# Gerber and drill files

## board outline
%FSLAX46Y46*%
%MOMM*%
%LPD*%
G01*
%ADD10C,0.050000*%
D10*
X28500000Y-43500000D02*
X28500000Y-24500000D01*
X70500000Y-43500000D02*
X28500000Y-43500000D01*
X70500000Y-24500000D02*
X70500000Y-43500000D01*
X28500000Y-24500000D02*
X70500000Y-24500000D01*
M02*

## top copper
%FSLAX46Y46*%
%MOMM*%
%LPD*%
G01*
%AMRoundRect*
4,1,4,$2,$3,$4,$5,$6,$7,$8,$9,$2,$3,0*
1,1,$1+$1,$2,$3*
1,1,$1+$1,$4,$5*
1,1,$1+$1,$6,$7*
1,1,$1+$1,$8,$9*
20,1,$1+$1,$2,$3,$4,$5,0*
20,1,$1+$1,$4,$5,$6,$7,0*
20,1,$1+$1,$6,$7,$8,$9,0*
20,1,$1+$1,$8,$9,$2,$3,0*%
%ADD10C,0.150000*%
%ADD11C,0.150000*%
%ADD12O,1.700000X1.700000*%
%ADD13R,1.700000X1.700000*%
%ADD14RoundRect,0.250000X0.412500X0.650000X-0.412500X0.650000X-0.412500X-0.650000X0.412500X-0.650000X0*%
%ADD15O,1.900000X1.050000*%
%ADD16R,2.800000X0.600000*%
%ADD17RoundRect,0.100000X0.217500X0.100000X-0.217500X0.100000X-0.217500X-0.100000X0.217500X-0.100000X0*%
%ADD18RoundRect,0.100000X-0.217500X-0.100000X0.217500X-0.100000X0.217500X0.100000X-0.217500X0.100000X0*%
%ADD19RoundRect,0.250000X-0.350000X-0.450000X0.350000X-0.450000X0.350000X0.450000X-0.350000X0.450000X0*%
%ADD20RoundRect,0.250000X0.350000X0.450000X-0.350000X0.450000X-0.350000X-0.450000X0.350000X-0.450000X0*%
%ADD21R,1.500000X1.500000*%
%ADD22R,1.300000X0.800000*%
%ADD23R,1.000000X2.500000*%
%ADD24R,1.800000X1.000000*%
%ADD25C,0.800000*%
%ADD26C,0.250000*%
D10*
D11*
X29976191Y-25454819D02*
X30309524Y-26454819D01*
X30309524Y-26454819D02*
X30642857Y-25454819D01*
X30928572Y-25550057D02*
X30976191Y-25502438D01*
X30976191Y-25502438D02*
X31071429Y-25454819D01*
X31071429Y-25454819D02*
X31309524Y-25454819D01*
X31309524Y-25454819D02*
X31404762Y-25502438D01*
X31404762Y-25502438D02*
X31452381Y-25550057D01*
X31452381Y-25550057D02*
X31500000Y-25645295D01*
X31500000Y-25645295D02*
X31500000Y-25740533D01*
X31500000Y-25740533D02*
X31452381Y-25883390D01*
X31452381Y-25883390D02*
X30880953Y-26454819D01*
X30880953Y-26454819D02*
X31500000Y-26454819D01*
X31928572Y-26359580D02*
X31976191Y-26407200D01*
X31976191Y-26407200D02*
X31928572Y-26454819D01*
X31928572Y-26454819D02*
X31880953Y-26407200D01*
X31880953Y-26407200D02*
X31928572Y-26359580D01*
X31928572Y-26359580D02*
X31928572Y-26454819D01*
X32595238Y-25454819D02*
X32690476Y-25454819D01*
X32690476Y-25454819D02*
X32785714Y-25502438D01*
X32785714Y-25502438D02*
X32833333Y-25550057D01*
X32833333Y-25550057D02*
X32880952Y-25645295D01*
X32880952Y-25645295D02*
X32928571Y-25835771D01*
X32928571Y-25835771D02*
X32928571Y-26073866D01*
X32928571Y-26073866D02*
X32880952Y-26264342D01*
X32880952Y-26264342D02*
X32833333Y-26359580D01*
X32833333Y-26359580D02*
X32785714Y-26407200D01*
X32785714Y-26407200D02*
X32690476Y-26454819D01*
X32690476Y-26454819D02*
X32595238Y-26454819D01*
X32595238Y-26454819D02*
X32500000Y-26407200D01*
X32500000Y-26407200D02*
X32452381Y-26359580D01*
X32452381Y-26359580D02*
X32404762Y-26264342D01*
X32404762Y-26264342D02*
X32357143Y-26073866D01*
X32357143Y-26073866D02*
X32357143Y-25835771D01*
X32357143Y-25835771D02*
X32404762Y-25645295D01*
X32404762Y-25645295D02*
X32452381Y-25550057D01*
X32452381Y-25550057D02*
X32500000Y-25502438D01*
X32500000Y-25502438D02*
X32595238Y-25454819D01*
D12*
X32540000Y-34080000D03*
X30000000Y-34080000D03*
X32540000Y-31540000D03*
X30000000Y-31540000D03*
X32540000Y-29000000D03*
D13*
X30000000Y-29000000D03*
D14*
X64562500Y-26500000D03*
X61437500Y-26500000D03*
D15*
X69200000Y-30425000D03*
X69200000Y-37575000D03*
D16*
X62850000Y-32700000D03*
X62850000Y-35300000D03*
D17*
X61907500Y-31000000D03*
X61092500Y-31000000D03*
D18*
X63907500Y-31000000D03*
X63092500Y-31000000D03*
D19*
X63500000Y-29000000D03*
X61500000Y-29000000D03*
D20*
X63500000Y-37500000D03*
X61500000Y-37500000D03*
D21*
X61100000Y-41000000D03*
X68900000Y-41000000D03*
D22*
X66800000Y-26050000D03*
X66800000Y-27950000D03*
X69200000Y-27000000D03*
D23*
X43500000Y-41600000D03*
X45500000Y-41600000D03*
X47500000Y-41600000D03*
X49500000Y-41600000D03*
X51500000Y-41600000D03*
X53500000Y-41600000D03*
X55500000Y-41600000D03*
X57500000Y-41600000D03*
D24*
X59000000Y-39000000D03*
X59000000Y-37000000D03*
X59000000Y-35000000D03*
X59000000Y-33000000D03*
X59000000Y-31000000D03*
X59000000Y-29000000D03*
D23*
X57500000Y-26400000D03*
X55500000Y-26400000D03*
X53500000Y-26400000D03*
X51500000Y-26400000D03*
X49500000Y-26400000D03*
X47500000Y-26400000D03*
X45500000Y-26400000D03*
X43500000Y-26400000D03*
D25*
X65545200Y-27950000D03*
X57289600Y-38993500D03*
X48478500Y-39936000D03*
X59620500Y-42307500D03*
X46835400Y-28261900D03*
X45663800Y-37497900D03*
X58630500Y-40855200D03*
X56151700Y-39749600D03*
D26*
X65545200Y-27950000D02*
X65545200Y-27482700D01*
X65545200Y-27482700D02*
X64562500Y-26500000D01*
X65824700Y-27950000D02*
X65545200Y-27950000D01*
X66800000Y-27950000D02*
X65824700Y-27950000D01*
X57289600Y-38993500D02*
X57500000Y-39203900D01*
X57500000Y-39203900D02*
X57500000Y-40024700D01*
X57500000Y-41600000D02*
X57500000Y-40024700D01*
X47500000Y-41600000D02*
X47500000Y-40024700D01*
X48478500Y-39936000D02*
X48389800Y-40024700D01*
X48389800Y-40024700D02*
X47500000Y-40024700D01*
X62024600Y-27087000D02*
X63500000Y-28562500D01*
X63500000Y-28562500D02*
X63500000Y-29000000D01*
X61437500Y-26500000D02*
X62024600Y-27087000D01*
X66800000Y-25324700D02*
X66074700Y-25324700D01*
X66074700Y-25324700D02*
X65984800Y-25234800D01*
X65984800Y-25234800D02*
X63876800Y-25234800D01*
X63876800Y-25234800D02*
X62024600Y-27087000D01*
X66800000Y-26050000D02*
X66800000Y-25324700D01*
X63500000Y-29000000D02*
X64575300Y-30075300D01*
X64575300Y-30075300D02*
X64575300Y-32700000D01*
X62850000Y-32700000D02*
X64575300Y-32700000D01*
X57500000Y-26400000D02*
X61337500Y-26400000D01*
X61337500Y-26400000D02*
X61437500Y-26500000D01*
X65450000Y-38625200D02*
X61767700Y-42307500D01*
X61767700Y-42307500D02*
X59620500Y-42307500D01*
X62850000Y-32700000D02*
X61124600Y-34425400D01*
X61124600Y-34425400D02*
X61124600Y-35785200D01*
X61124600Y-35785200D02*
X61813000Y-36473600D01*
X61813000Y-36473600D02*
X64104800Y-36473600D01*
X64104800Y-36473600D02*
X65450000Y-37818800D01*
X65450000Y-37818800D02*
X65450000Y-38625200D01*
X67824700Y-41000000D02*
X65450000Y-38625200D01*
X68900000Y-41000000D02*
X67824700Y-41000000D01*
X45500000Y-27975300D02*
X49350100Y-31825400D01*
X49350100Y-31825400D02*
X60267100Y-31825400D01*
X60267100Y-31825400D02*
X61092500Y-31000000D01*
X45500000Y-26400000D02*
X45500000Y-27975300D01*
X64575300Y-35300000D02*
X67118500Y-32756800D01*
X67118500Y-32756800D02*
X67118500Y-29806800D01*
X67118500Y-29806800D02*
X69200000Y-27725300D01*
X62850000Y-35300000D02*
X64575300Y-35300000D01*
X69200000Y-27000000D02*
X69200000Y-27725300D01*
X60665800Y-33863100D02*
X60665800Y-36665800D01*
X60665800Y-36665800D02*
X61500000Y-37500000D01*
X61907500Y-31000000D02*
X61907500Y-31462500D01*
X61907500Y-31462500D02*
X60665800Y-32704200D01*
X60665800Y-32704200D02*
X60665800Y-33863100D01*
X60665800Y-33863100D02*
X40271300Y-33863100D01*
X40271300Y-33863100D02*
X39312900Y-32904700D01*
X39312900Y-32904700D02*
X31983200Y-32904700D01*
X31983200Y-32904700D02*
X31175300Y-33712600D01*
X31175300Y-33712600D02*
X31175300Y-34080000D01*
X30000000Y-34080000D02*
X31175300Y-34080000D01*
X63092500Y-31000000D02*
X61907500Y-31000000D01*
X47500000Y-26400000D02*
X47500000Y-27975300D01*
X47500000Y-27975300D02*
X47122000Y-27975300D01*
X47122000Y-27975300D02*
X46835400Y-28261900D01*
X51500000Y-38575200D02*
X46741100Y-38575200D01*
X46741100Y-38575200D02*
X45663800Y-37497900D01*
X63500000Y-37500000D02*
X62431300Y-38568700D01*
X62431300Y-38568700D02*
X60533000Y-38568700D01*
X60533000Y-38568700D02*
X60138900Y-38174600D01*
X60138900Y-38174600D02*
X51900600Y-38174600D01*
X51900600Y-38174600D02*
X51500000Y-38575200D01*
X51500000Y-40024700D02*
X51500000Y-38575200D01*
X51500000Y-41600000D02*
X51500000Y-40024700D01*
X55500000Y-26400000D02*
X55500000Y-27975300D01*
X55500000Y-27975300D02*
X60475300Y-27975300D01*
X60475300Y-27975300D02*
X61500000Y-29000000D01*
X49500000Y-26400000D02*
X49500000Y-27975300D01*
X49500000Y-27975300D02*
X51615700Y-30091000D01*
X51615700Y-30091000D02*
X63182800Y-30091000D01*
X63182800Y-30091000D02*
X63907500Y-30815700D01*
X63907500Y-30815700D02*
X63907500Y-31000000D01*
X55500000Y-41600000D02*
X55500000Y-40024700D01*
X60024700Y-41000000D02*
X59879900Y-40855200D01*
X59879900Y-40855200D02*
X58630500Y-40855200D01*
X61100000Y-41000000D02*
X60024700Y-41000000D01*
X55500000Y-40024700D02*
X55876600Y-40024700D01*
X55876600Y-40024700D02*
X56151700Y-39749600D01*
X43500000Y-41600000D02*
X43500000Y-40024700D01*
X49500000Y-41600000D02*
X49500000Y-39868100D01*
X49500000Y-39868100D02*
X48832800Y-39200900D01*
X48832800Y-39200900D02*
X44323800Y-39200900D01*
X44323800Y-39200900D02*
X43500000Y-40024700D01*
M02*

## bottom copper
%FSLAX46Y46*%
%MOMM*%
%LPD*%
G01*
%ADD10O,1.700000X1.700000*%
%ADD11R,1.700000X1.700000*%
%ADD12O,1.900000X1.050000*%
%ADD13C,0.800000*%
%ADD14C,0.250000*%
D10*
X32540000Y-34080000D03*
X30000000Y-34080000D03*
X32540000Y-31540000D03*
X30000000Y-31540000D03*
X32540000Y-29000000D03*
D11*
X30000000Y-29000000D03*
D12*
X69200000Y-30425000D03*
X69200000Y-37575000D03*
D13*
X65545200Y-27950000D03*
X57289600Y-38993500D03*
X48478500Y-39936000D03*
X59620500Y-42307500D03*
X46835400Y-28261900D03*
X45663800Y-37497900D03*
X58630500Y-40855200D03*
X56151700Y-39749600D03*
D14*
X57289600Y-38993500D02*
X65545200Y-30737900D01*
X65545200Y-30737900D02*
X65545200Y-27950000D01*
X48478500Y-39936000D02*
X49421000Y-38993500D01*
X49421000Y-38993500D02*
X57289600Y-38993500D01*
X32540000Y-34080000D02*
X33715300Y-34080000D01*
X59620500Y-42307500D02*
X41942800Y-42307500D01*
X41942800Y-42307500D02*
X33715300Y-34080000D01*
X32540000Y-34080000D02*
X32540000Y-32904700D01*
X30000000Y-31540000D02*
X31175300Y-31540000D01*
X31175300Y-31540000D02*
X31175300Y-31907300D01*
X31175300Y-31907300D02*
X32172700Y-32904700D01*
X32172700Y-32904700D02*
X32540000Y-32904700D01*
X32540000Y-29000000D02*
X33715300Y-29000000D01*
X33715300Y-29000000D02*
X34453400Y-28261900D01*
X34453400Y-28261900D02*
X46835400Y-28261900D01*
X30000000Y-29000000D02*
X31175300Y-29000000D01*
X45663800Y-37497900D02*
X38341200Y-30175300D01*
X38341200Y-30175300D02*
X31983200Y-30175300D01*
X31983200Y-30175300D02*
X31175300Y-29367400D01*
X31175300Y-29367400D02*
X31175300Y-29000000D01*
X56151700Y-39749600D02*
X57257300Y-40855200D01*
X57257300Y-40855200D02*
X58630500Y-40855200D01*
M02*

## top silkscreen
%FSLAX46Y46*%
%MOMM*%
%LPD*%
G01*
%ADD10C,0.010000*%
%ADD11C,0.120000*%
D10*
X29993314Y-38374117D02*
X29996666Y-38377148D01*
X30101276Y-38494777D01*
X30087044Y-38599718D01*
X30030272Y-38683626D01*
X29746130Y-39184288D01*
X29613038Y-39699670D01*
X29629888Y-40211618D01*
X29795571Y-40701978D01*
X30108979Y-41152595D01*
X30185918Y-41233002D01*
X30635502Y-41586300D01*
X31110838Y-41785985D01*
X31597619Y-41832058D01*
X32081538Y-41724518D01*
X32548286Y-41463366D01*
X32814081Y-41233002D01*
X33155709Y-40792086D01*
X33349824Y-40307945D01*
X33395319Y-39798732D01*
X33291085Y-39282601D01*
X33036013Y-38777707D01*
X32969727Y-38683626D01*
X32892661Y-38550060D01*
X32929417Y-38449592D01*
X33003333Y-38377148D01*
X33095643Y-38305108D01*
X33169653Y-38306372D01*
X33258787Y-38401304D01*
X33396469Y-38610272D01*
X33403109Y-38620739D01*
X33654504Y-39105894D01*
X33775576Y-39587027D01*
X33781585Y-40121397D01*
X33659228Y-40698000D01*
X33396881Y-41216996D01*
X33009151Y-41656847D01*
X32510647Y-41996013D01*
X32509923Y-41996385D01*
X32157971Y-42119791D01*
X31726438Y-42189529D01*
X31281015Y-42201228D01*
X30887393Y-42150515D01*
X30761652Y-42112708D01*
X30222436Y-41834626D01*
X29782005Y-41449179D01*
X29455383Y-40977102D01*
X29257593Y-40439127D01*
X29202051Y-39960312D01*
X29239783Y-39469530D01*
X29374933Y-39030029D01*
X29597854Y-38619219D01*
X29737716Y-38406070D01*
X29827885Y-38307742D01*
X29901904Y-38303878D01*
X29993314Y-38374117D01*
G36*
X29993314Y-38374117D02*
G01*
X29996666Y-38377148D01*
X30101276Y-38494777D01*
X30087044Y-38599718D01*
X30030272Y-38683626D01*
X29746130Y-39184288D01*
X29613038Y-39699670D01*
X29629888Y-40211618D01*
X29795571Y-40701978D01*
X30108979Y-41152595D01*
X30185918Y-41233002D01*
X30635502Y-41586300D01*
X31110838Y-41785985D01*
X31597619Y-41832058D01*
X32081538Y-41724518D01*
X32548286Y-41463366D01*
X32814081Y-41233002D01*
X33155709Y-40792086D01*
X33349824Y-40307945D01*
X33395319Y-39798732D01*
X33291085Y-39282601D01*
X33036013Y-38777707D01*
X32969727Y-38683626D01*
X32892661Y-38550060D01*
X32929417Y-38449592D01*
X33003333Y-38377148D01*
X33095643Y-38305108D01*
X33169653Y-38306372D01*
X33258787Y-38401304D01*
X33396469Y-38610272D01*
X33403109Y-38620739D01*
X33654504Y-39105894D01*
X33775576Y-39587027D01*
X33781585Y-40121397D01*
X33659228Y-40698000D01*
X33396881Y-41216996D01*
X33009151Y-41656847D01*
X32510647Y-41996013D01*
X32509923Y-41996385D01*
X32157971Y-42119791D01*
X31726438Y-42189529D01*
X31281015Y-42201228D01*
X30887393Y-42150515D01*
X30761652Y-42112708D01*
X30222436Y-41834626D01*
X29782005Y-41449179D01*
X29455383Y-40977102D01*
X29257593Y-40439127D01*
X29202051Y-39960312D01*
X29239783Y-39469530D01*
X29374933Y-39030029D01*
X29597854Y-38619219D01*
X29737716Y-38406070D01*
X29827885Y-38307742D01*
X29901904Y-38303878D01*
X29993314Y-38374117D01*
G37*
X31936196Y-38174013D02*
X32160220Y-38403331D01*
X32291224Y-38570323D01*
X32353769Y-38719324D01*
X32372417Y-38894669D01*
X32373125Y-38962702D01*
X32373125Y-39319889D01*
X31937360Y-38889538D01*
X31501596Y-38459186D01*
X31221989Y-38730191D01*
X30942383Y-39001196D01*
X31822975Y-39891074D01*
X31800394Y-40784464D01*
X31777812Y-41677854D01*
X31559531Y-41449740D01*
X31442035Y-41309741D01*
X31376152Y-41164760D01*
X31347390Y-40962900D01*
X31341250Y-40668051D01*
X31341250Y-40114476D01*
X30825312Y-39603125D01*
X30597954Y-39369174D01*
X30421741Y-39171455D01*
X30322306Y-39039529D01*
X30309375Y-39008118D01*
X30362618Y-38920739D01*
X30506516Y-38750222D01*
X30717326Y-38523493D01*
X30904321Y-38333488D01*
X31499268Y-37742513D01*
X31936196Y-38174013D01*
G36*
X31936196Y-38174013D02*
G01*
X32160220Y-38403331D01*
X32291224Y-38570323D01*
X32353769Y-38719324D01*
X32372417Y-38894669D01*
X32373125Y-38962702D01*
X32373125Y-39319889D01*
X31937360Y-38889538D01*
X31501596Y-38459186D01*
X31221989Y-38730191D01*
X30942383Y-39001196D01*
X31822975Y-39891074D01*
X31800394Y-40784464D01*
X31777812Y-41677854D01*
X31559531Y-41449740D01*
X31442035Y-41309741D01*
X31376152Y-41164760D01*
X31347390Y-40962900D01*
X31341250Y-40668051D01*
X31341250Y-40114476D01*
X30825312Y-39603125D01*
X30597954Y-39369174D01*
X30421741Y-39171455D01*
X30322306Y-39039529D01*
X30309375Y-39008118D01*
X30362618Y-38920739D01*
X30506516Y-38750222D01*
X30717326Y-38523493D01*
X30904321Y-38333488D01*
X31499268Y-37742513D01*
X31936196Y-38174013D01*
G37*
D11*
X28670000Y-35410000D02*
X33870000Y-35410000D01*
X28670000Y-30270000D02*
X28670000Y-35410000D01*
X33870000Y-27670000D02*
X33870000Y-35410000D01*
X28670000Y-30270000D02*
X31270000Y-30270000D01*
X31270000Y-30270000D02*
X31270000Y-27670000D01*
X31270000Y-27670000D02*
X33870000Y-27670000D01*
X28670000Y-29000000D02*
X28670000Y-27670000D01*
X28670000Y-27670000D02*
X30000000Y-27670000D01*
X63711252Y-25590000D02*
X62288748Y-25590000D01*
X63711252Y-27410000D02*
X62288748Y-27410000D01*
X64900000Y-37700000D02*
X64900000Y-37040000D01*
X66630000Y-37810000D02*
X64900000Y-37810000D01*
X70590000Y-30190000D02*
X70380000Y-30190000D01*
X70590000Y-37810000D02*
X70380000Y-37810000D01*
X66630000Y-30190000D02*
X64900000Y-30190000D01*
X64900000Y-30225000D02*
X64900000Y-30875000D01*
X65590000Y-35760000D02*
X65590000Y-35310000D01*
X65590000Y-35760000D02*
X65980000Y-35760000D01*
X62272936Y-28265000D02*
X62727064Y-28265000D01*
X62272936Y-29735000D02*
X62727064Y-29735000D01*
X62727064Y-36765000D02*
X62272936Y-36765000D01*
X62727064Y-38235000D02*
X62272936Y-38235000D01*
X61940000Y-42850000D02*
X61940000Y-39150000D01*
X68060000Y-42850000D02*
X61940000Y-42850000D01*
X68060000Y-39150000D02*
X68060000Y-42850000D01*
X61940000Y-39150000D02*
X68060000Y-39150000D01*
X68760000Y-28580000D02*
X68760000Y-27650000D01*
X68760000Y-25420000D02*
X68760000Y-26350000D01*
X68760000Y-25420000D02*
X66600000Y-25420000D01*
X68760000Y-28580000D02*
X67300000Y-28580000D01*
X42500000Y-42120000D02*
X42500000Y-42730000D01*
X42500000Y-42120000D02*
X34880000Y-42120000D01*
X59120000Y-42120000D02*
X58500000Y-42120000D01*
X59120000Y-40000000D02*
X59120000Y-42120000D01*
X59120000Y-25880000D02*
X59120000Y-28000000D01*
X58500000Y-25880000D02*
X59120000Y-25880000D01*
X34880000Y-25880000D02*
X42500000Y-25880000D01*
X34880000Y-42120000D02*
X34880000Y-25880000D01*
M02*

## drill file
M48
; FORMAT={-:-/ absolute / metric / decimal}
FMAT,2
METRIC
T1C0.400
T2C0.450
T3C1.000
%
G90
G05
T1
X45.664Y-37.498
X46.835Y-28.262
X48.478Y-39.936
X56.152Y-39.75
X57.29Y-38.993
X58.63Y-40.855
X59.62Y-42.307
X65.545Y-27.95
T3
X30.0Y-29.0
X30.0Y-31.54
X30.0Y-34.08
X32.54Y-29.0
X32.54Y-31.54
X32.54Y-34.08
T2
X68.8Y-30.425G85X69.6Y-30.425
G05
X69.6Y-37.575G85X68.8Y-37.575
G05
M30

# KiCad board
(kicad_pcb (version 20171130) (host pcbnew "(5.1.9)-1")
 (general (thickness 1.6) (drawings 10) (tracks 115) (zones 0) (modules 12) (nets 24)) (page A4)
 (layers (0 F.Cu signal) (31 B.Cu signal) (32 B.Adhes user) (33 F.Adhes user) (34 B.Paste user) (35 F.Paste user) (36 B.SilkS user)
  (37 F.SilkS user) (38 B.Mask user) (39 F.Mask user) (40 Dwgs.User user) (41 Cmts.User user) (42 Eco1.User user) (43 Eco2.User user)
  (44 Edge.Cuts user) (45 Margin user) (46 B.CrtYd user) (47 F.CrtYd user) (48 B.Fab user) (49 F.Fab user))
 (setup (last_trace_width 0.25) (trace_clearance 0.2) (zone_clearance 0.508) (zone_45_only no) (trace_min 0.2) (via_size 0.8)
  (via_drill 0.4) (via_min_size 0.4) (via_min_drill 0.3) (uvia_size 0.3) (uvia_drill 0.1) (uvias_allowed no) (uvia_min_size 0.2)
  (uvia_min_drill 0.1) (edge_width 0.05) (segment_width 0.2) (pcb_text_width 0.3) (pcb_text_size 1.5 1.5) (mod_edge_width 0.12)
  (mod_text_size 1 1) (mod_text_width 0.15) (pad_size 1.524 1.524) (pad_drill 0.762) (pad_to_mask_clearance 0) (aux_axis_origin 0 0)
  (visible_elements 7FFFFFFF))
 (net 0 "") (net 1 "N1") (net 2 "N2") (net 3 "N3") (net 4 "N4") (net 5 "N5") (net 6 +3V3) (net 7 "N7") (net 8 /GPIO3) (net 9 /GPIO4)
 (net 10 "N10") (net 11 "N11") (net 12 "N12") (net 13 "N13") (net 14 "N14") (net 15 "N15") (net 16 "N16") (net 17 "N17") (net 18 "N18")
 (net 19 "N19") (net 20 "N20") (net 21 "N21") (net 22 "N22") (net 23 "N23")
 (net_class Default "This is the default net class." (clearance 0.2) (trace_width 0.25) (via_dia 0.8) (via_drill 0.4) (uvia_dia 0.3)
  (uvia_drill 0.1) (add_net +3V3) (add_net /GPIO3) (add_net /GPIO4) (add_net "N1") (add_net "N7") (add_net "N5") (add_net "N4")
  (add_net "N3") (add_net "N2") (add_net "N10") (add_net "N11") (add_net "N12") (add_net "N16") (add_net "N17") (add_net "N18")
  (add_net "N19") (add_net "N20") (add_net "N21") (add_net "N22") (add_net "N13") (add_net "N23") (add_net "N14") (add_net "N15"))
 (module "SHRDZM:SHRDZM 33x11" (layer B.Cu) (at 51 31.5 180)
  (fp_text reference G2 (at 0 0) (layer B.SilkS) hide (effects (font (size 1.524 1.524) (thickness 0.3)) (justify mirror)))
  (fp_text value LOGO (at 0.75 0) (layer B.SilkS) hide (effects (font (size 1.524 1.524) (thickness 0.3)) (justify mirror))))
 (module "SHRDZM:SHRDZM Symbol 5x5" (layer F.Cu) (at 31.5 40)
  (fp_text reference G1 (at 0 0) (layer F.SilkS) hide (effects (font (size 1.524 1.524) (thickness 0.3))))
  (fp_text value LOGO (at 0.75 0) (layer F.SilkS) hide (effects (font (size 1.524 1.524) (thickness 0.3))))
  (fp_poly
   (pts (xy -1.506686 -1.625883) (xy -1.503334 -1.622852) (xy -1.398724 -1.505223) (xy -1.412956 -1.400282) (xy -1.469728 -1.316374)
    (xy -1.75387 -0.815712) (xy -1.886962 -0.30033) (xy -1.870112 0.211618) (xy -1.704429 0.701978) (xy -1.391021 1.152595)
    (xy -1.314082 1.233002) (xy -0.864498 1.5863) (xy -0.389162 1.785985) (xy 0.097619 1.832058) (xy 0.581538 1.724518)
    (xy 1.048286 1.463366) (xy 1.314081 1.233002) (xy 1.655709 0.792086) (xy 1.849824 0.307945) (xy 1.895319 -0.201268)
    (xy 1.791085 -0.717399) (xy 1.536013 -1.222293) (xy 1.469727 -1.316374) (xy 1.392661 -1.44994) (xy 1.429417 -1.550408)
    (xy 1.503333 -1.622852) (xy 1.595643 -1.694892) (xy 1.669653 -1.693628) (xy 1.758787 -1.598696) (xy 1.896469 -1.389728)
    (xy 1.903109 -1.379261) (xy 2.154504 -0.894106) (xy 2.275576 -0.412973) (xy 2.281585 0.121397) (xy 2.159228 0.698)
    (xy 1.896881 1.216996) (xy 1.509151 1.656847) (xy 1.010647 1.996013) (xy 1.009923 1.996385) (xy 0.657971 2.119791)
    (xy 0.226438 2.189529) (xy -0.218985 2.201228) (xy -0.612607 2.150515) (xy -0.738348 2.112708) (xy -1.277564 1.834626)
    (xy -1.717995 1.449179) (xy -2.044617 0.977102) (xy -2.242407 0.439127) (xy -2.297949 -0.039688) (xy -2.260217 -0.53047)
    (xy -2.125067 -0.969971) (xy -1.902146 -1.380781) (xy -1.762284 -1.59393) (xy -1.672115 -1.692258) (xy -1.598096 -1.696122)
    (xy -1.506686 -1.625883))
   (layer F.SilkS) (width 0.01))
  (fp_poly
   (pts (xy 0.436196 -1.825987) (xy 0.66022 -1.596669) (xy 0.791224 -1.429677) (xy 0.853769 -1.280676) (xy 0.872417 -1.105331)
    (xy 0.873125 -1.037298) (xy 0.873125 -0.680111) (xy 0.43736 -1.110462) (xy 0.001596 -1.540814) (xy -0.278011 -1.269809)
    (xy -0.557617 -0.998804) (xy 0.322975 -0.108926) (xy 0.300394 0.784464) (xy 0.277812 1.677854) (xy 0.059531 1.44974)
    (xy -0.057965 1.309741) (xy -0.123848 1.16476) (xy -0.15261 0.9629) (xy -0.15875 0.668051) (xy -0.15875 0.114476)
    (xy -0.674688 -0.396875) (xy -0.902046 -0.630826) (xy -1.078259 -0.828545) (xy -1.177694 -0.960471) (xy -1.190625 -0.991882)
    (xy -1.137382 -1.079261) (xy -0.993484 -1.249778) (xy -0.782674 -1.476507) (xy -0.595679 -1.666512) (xy -0.000732 -2.257487)
    (xy 0.436196 -1.825987))
   (layer F.SilkS) (width 0.01)))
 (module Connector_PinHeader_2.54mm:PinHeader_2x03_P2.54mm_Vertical (layer F.Cu) (at 30 29)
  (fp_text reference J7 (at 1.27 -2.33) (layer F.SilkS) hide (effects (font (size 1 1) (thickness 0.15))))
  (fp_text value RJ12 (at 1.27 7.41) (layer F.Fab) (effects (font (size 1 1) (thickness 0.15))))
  (fp_line (start -1.33 6.41) (end 3.87 6.41) (layer F.SilkS) (width 0.12))
  (fp_line (start -1.33 1.27) (end -1.33 6.41) (layer F.SilkS) (width 0.12))
  (fp_line (start 3.87 -1.33) (end 3.87 6.41) (layer F.SilkS) (width 0.12))
  (fp_line (start -1.33 1.27) (end 1.27 1.27) (layer F.SilkS) (width 0.12))
  (fp_line (start 1.27 1.27) (end 1.27 -1.33) (layer F.SilkS) (width 0.12))
  (fp_line (start 1.27 -1.33) (end 3.87 -1.33) (layer F.SilkS) (width 0.12))
  (fp_line (start -1.33 0) (end -1.33 -1.33) (layer F.SilkS) (width 0.12))
  (fp_line (start -1.33 -1.33) (end 0 -1.33) (layer F.SilkS) (width 0.12))
  (pad 6 thru_hole oval (at 2.54 5.08) (size 1.7 1.7) (drill 1) (layers *.Cu *.Mask) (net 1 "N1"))
  (pad 5 thru_hole oval (at 0 5.08) (size 1.7 1.7) (drill 1) (layers *.Cu *.Mask) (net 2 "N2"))
  (pad 4 thru_hole oval (at 2.54 2.54) (size 1.7 1.7) (drill 1) (layers *.Cu *.Mask) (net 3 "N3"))
  (pad 3 thru_hole oval (at 0 2.54) (size 1.7 1.7) (drill 1) (layers *.Cu *.Mask) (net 1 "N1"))
  (pad 2 thru_hole oval (at 2.54 0) (size 1.7 1.7) (drill 1) (layers *.Cu *.Mask) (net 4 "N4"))
  (pad 1 thru_hole rect (at 0 0) (size 1.7 1.7) (drill 1) (layers *.Cu *.Mask) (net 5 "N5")))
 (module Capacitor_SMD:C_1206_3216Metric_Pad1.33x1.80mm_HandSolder (layer F.Cu) (at 63 26.5 180)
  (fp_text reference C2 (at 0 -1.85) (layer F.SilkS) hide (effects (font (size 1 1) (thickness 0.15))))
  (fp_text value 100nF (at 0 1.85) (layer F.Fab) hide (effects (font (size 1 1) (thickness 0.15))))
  (fp_line (start -0.711252 0.91) (end 0.711252 0.91) (layer F.SilkS) (width 0.12))
  (fp_line (start -0.711252 -0.91) (end 0.711252 -0.91) (layer F.SilkS) (width 0.12))
  (pad 1 smd roundrect (at -1.5625 0 180) (size 1.325 1.8) (layers F.Cu F.Paste F.Mask) (roundrect_rratio 0.188679) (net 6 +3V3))
  (pad 2 smd roundrect (at 1.5625 0 180) (size 1.325 1.8) (layers F.Cu F.Paste F.Mask) (roundrect_rratio 0.188679) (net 1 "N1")))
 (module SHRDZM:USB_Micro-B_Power (layer F.Cu) (at 68 34 90)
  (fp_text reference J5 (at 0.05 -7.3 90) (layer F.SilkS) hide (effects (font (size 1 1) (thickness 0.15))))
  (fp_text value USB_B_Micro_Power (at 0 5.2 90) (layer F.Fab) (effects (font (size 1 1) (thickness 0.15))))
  (fp_line (start -3.7 -3.1) (end -3.04 -3.1) (layer F.SilkS) (width 0.12))
  (fp_line (start -3.81 -1.37) (end -3.81 -3.1) (layer F.SilkS) (width 0.12))
  (fp_line (start 3.81 2.59) (end 3.81 2.38) (layer F.SilkS) (width 0.12))
  (fp_line (start -3.81 2.59) (end -3.81 2.38) (layer F.SilkS) (width 0.12))
  (fp_line (start 3.81 -1.37) (end 3.81 -3.1) (layer F.SilkS) (width 0.12))
  (fp_line (start 3.775 -3.1) (end 3.125 -3.1) (layer F.SilkS) (width 0.12))
  (fp_line (start -1.76 -2.41) (end -1.31 -2.41) (layer F.SilkS) (width 0.12))
  (fp_line (start -1.76 -2.41) (end -1.76 -2.02) (layer F.SilkS) (width 0.12))
  (pad "" thru_hole oval (at 3.575 1.2 90) (size 1.05 1.9) (drill oval 0.45 1.25) (layers *.Cu *.Mask))
  (pad "" thru_hole oval (at -3.575 1.2 270) (size 1.05 1.9) (drill oval 0.45 1.25) (layers *.Cu *.Mask))
  (pad 5 smd rect (at 1.3 -5.15 90) (size 0.6 2.8) (layers F.Cu F.Paste F.Mask) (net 1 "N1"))
  (pad 1 smd rect (at -1.3 -5.15 90) (size 0.6 2.8) (layers F.Cu F.Paste F.Mask) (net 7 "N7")))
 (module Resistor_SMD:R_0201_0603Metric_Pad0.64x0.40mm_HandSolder (layer F.Cu) (at 61.5 31 180)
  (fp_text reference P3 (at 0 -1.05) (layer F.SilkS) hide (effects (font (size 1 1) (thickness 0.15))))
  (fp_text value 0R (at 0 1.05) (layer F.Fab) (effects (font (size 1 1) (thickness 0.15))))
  (pad "" smd roundrect (at -0.4325 0 180) (size 0.458 0.36) (layers F.Paste) (roundrect_rratio 0.25))
  (pad "" smd roundrect (at 0.4325 0 180) (size 0.458 0.36) (layers F.Paste) (roundrect_rratio 0.25))
  (pad 1 smd roundrect (at -0.4075 0 180) (size 0.635 0.4) (layers F.Cu F.Mask) (roundrect_rratio 0.25) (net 2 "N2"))
  (pad 2 smd roundrect (at 0.4075 0 180) (size 0.635 0.4) (layers F.Cu F.Mask) (roundrect_rratio 0.25) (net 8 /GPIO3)))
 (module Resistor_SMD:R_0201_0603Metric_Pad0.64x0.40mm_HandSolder (layer F.Cu) (at 63.5 31)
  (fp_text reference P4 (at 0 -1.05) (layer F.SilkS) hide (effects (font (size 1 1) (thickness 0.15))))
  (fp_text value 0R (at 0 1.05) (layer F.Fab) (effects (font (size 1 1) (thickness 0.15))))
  (pad 2 smd roundrect (at 0.4075 0) (size 0.635 0.4) (layers F.Cu F.Mask) (roundrect_rratio 0.25) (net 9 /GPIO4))
  (pad 1 smd roundrect (at -0.4075 0) (size 0.635 0.4) (layers F.Cu F.Mask) (roundrect_rratio 0.25) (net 2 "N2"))
  (pad "" smd roundrect (at 0.4325 0) (size 0.458 0.36) (layers F.Paste) (roundrect_rratio 0.25))
  (pad "" smd roundrect (at -0.4325 0) (size 0.458 0.36) (layers F.Paste) (roundrect_rratio 0.25)))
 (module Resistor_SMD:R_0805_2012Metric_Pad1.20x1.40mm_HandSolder (layer F.Cu) (at 62.5 29)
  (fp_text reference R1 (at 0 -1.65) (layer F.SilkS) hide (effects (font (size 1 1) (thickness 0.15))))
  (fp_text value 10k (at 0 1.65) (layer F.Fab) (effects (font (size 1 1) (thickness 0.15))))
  (fp_line (start -0.227064 -0.735) (end 0.227064 -0.735) (layer F.SilkS) (width 0.12))
  (fp_line (start -0.227064 0.735) (end 0.227064 0.735) (layer F.SilkS) (width 0.12))
  (pad 2 smd roundrect (at 1 0) (size 1.2 1.4) (layers F.Cu F.Paste F.Mask) (roundrect_rratio 0.208333) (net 1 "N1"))
  (pad 1 smd roundrect (at -1 0) (size 1.2 1.4) (layers F.Cu F.Paste F.Mask) (roundrect_rratio 0.208333) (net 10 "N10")))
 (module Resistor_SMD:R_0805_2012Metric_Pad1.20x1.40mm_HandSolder (layer F.Cu) (at 62.5 37.5 180)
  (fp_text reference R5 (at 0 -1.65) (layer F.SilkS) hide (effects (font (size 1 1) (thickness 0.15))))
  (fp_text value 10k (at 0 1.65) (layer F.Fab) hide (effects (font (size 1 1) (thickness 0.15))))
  (fp_line (start -0.227064 0.735) (end 0.227064 0.735) (layer F.SilkS) (width 0.12))
  (fp_line (start -0.227064 -0.735) (end 0.227064 -0.735) (layer F.SilkS) (width 0.12))
  (pad 1 smd roundrect (at -1 0 180) (size 1.2 1.4) (layers F.Cu F.Paste F.Mask) (roundrect_rratio 0.208333) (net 5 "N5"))
  (pad 2 smd roundrect (at 1 0 180) (size 1.2 1.4) (layers F.Cu F.Paste F.Mask) (roundrect_rratio 0.208333) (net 2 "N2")))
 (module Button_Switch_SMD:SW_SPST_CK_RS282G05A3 (layer F.Cu) (at 65 41)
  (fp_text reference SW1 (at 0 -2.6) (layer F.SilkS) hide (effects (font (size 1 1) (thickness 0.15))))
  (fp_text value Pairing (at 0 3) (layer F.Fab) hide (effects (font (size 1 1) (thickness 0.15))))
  (fp_line (start -3.06 1.85) (end -3.06 -1.85) (layer F.SilkS) (width 0.12))
  (fp_line (start 3.06 1.85) (end -3.06 1.85) (layer F.SilkS) (width 0.12))
  (fp_line (start 3.06 -1.85) (end 3.06 1.85) (layer F.SilkS) (width 0.12))
  (fp_line (start -3.06 -1.85) (end 3.06 -1.85) (layer F.SilkS) (width 0.12))
  (pad 1 smd rect (at -3.9 0) (size 1.5 1.5) (layers F.Cu F.Paste F.Mask) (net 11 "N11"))
  (pad 2 smd rect (at 3.9 0) (size 1.5 1.5) (layers F.Cu F.Paste F.Mask) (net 1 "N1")))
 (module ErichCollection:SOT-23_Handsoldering (layer F.Cu) (at 68 27)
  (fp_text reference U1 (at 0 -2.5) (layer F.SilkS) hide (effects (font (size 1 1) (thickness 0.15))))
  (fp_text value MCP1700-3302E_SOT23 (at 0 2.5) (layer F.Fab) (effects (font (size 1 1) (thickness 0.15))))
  (fp_line (start 0.76 1.58) (end 0.76 0.65) (layer F.SilkS) (width 0.12))
  (fp_line (start 0.76 -1.58) (end 0.76 -0.65) (layer F.SilkS) (width 0.12))
  (fp_line (start 0.76 -1.58) (end -1.4 -1.58) (layer F.SilkS) (width 0.12))
  (fp_line (start 0.76 1.58) (end -0.7 1.58) (layer F.SilkS) (width 0.12))
  (pad 1 smd rect (at -1.2 -0.95) (size 1.3 0.8) (layers F.Cu F.Paste F.Mask) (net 1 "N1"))
  (pad 2 smd rect (at -1.2 0.95) (size 1.3 0.8) (layers F.Cu F.Paste F.Mask) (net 6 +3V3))
  (pad 3 smd rect (at 1.2 0) (size 1.3 0.8) (layers F.Cu F.Paste F.Mask) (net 7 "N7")))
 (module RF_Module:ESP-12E (layer F.Cu) (at 47 34 90)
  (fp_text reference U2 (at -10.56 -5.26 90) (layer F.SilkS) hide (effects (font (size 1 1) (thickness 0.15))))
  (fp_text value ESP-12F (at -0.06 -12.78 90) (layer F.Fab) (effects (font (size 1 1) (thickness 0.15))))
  (fp_line (start -8.12 -4.5) (end -8.73 -4.5) (layer F.SilkS) (width 0.12))
  (fp_line (start -8.12 -4.5) (end -8.12 -12.12) (layer F.SilkS) (width 0.12))
  (fp_line (start -8.12 12.12) (end -8.12 11.5) (layer F.SilkS) (width 0.12))
  (fp_line (start -6 12.12) (end -8.12 12.12) (layer F.SilkS) (width 0.12))
  (fp_line (start 8.12 12.12) (end 6 12.12) (layer F.SilkS) (width 0.12))
  (fp_line (start 8.12 11.5) (end 8.12 12.12) (layer F.SilkS) (width 0.12))
  (fp_line (start 8.12 -12.12) (end 8.12 -4.5) (layer F.SilkS) (width 0.12))
  (fp_line (start -8.12 -12.12) (end 8.12 -12.12) (layer F.SilkS) (width 0.12))
  (pad 1 smd rect (at -7.6 -3.5 90) (size 2.5 1) (layers F.Cu F.Paste F.Mask) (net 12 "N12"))
  (pad 2 smd rect (at -7.6 -1.5 90) (size 2.5 1) (layers F.Cu F.Paste F.Mask) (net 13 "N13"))
  (pad 3 smd rect (at -7.6 0.5 90) (size 2.5 1) (layers F.Cu F.Paste F.Mask) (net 6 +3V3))
  (pad 4 smd rect (at -7.6 2.5 90) (size 2.5 1) (layers F.Cu F.Paste F.Mask) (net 12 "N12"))
  (pad 5 smd rect (at -7.6 4.5 90) (size 2.5 1) (layers F.Cu F.Paste F.Mask) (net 5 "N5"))
  (pad 6 smd rect (at -7.6 6.5 90) (size 2.5 1) (layers F.Cu F.Paste F.Mask) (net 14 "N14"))
  (pad 7 smd rect (at -7.6 8.5 90) (size 2.5 1) (layers F.Cu F.Paste F.Mask) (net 11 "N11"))
  (pad 8 smd rect (at -7.6 10.5 90) (size 2.5 1) (layers F.Cu F.Paste F.Mask) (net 6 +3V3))
  (pad 9 smd rect (at -5 12 90) (size 1 1.8) (layers F.Cu F.Paste F.Mask) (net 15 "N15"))
  (pad 10 smd rect (at -3 12 90) (size 1 1.8) (layers F.Cu F.Paste F.Mask) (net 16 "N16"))
  (pad 11 smd rect (at -1 12 90) (size 1 1.8) (layers F.Cu F.Paste F.Mask) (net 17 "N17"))
  (pad 12 smd rect (at 1 12 90) (size 1 1.8) (layers F.Cu F.Paste F.Mask) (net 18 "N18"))
  (pad 13 smd rect (at 3 12 90) (size 1 1.8) (layers F.Cu F.Paste F.Mask) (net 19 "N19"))
  (pad 14 smd rect (at 5 12 90) (size 1 1.8) (layers F.Cu F.Paste F.Mask) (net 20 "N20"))
  (pad 15 smd rect (at 7.6 10.5 90) (size 2.5 1) (layers F.Cu F.Paste F.Mask) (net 1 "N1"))
  (pad 16 smd rect (at 7.6 8.5 90) (size 2.5 1) (layers F.Cu F.Paste F.Mask) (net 10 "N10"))
  (pad 17 smd rect (at 7.6 6.5 90) (size 2.5 1) (layers F.Cu F.Paste F.Mask) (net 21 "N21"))
  (pad 18 smd rect (at 7.6 4.5 90) (size 2.5 1) (layers F.Cu F.Paste F.Mask) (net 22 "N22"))
  (pad 19 smd rect (at 7.6 2.5 90) (size 2.5 1) (layers F.Cu F.Paste F.Mask) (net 9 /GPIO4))
  (pad 20 smd rect (at 7.6 0.5 90) (size 2.5 1) (layers F.Cu F.Paste F.Mask) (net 4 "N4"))
  (pad 21 smd rect (at 7.6 -1.5 90) (size 2.5 1) (layers F.Cu F.Paste F.Mask) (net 8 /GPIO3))
  (pad 22 smd rect (at 7.6 -3.5 90) (size 2.5 1) (layers F.Cu F.Paste F.Mask) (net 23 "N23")))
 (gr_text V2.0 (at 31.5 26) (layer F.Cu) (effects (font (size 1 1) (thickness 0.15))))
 (gr_line (start 28.5 43.5) (end 28.5 24.5) (layer Edge.Cuts) (width 0.05))
 (gr_line (start 70.5 43.5) (end 28.5 43.5) (layer Edge.Cuts) (width 0.05))
 (gr_line (start 70.5 24.5) (end 70.5 43.5) (layer Edge.Cuts) (width 0.05))
 (gr_line (start 28.5 24.5) (end 70.5 24.5) (layer Edge.Cuts) (width 0.05))
 (segment (start 65.5452 27.95) (end 65.5452 27.4827) (width 0.25) (layer F.Cu) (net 6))
 (segment (start 65.5452 27.4827) (end 64.5625 26.5) (width 0.25) (layer F.Cu) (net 6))
 (segment (start 65.8247 27.95) (end 65.5452 27.95) (width 0.25) (layer F.Cu) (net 6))
 (segment (start 57.2896 38.9935) (end 65.5452 30.7379) (width 0.25) (layer B.Cu) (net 6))
 (segment (start 65.5452 30.7379) (end 65.5452 27.95) (width 0.25) (layer B.Cu) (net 6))
 (segment (start 66.8 27.95) (end 65.8247 27.95) (width 0.25) (layer F.Cu) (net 6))
 (segment (start 57.2896 38.9935) (end 57.5 39.2039) (width 0.25) (layer F.Cu) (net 6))
 (segment (start 57.5 39.2039) (end 57.5 40.0247) (width 0.25) (layer F.Cu) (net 6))
 (segment (start 48.4785 39.936) (end 49.421 38.9935) (width 0.25) (layer B.Cu) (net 6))
 (segment (start 49.421 38.9935) (end 57.2896 38.9935) (width 0.25) (layer B.Cu) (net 6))
 (segment (start 57.5 41.6) (end 57.5 40.0247) (width 0.25) (layer F.Cu) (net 6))
 (segment (start 47.5 41.6) (end 47.5 40.0247) (width 0.25) (layer F.Cu) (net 6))
 (segment (start 48.4785 39.936) (end 48.3898 40.0247) (width 0.25) (layer F.Cu) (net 6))
 (segment (start 48.3898 40.0247) (end 47.5 40.0247) (width 0.25) (layer F.Cu) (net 6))
 (via (at 65.5452 27.95) (size 0.8) (layers F.Cu B.Cu) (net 6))
 (via (at 57.2896 38.9935) (size 0.8) (layers F.Cu B.Cu) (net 6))
 (via (at 48.4785 39.936) (size 0.8) (layers F.Cu B.Cu) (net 6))
 (segment (start 62.0246 27.087) (end 63.5 28.5625) (width 0.25) (layer F.Cu) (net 1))
 (segment (start 63.5 28.5625) (end 63.5 29) (width 0.25) (layer F.Cu) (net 1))
 (segment (start 61.4375 26.5) (end 62.0246 27.087) (width 0.25) (layer F.Cu) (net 1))
 (segment (start 66.8 25.3247) (end 66.0747 25.3247) (width 0.25) (layer F.Cu) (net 1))
 (segment (start 66.0747 25.3247) (end 65.9848 25.2348) (width 0.25) (layer F.Cu) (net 1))
 (segment (start 65.9848 25.2348) (end 63.8768 25.2348) (width 0.25) (layer F.Cu) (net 1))
 (segment (start 63.8768 25.2348) (end 62.0246 27.087) (width 0.25) (layer F.Cu) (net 1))
 (segment (start 66.8 26.05) (end 66.8 25.3247) (width 0.25) (layer F.Cu) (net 1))
 (segment (start 63.5 29) (end 64.5753 30.0753) (width 0.25) (layer F.Cu) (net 1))
 (segment (start 64.5753 30.0753) (end 64.5753 32.7) (width 0.25) (layer F.Cu) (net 1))
 (segment (start 62.85 32.7) (end 64.5753 32.7) (width 0.25) (layer F.Cu) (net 1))
 (segment (start 57.5 26.4) (end 61.3375 26.4) (width 0.25) (layer F.Cu) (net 1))
 (segment (start 61.3375 26.4) (end 61.4375 26.5) (width 0.25) (layer F.Cu) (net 1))
 (segment (start 65.45 38.6252) (end 61.7677 42.3075) (width 0.25) (layer F.Cu) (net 1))
 (segment (start 61.7677 42.3075) (end 59.6205 42.3075) (width 0.25) (layer F.Cu) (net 1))
 (segment (start 62.85 32.7) (end 61.1246 34.4254) (width 0.25) (layer F.Cu) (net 1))
 (segment (start 61.1246 34.4254) (end 61.1246 35.7852) (width 0.25) (layer F.Cu) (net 1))
 (segment (start 61.1246 35.7852) (end 61.813 36.4736) (width 0.25) (layer F.Cu) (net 1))
 (segment (start 61.813 36.4736) (end 64.1048 36.4736) (width 0.25) (layer F.Cu) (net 1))
 (segment (start 64.1048 36.4736) (end 65.45 37.8188) (width 0.25) (layer F.Cu) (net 1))
 (segment (start 65.45 37.8188) (end 65.45 38.6252) (width 0.25) (layer F.Cu) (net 1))
 (segment (start 67.8247 41) (end 65.45 38.6252) (width 0.25) (layer F.Cu) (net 1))
 (segment (start 32.54 34.08) (end 33.7153 34.08) (width 0.25) (layer B.Cu) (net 1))
 (segment (start 59.6205 42.3075) (end 41.9428 42.3075) (width 0.25) (layer B.Cu) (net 1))
 (segment (start 41.9428 42.3075) (end 33.7153 34.08) (width 0.25) (layer B.Cu) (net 1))
 (segment (start 68.9 41) (end 67.8247 41) (width 0.25) (layer F.Cu) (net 1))
 (segment (start 32.54 34.08) (end 32.54 32.9047) (width 0.25) (layer B.Cu) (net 1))
 (segment (start 30 31.54) (end 31.1753 31.54) (width 0.25) (layer B.Cu) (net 1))
 (segment (start 31.1753 31.54) (end 31.1753 31.9073) (width 0.25) (layer B.Cu) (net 1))
 (segment (start 31.1753 31.9073) (end 32.1727 32.9047) (width 0.25) (layer B.Cu) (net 1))
 (segment (start 32.1727 32.9047) (end 32.54 32.9047) (width 0.25) (layer B.Cu) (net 1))
 (via (at 59.6205 42.3075) (size 0.8) (layers F.Cu B.Cu) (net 1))
 (segment (start 45.5 27.9753) (end 49.3501 31.8254) (width 0.25) (layer F.Cu) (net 8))
 (segment (start 49.3501 31.8254) (end 60.2671 31.8254) (width 0.25) (layer F.Cu) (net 8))
 (segment (start 60.2671 31.8254) (end 61.0925 31) (width 0.25) (layer F.Cu) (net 8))
 (segment (start 45.5 26.4) (end 45.5 27.9753) (width 0.25) (layer F.Cu) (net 8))
 (segment (start 64.5753 35.3) (end 67.1185 32.7568) (width 0.25) (layer F.Cu) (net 7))
 (segment (start 67.1185 32.7568) (end 67.1185 29.8068) (width 0.25) (layer F.Cu) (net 7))
 (segment (start 67.1185 29.8068) (end 69.2 27.7253) (width 0.25) (layer F.Cu) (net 7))
 (segment (start 62.85 35.3) (end 64.5753 35.3) (width 0.25) (layer F.Cu) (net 7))
 (segment (start 69.2 27) (end 69.2 27.7253) (width 0.25) (layer F.Cu) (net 7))
 (segment (start 60.6658 33.8631) (end 60.6658 36.6658) (width 0.25) (layer F.Cu) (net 2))
 (segment (start 60.6658 36.6658) (end 61.5 37.5) (width 0.25) (layer F.Cu) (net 2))
 (segment (start 61.9075 31) (end 61.9075 31.4625) (width 0.25) (layer F.Cu) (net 2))
 (segment (start 61.9075 31.4625) (end 60.6658 32.7042) (width 0.25) (layer F.Cu) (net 2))
 (segment (start 60.6658 32.7042) (end 60.6658 33.8631) (width 0.25) (layer F.Cu) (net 2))
 (segment (start 60.6658 33.8631) (end 40.2713 33.8631) (width 0.25) (layer F.Cu) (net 2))
 (segment (start 40.2713 33.8631) (end 39.3129 32.9047) (width 0.25) (layer F.Cu) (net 2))
 (segment (start 39.3129 32.9047) (end 31.9832 32.9047) (width 0.25) (layer F.Cu) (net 2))
 (segment (start 31.9832 32.9047) (end 31.1753 33.7126) (width 0.25) (layer F.Cu) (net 2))
 (segment (start 31.1753 33.7126) (end 31.1753 34.08) (width 0.25) (layer F.Cu) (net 2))
 (segment (start 30 34.08) (end 31.1753 34.08) (width 0.25) (layer F.Cu) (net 2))
 (segment (start 63.0925 31) (end 61.9075 31) (width 0.25) (layer F.Cu) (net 2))
 (segment (start 47.5 26.4) (end 47.5 27.9753) (width 0.25) (layer F.Cu) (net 4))
 (segment (start 32.54 29) (end 33.7153 29) (width 0.25) (layer B.Cu) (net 4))
 (segment (start 47.5 27.9753) (end 47.122 27.9753) (width 0.25) (layer F.Cu) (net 4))
 (segment (start 47.122 27.9753) (end 46.8354 28.2619) (width 0.25) (layer F.Cu) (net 4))
 (segment (start 33.7153 29) (end 34.4534 28.2619) (width 0.25) (layer B.Cu) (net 4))
 (segment (start 34.4534 28.2619) (end 46.8354 28.2619) (width 0.25) (layer B.Cu) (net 4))
 (via (at 46.8354 28.2619) (size 0.8) (layers F.Cu B.Cu) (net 4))
 (segment (start 30 29) (end 31.1753 29) (width 0.25) (layer B.Cu) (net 5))
 (segment (start 51.5 38.5752) (end 46.7411 38.5752) (width 0.25) (layer F.Cu) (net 5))
 (segment (start 46.7411 38.5752) (end 45.6638 37.4979) (width 0.25) (layer F.Cu) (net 5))
 (segment (start 63.5 37.5) (end 62.4313 38.5687) (width 0.25) (layer F.Cu) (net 5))
 (segment (start 62.4313 38.5687) (end 60.533 38.5687) (width 0.25) (layer F.Cu) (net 5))
 (segment (start 60.533 38.5687) (end 60.1389 38.1746) (width 0.25) (layer F.Cu) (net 5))
 (segment (start 60.1389 38.1746) (end 51.9006 38.1746) (width 0.25) (layer F.Cu) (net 5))
 (segment (start 51.9006 38.1746) (end 51.5 38.5752) (width 0.25) (layer F.Cu) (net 5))
 (segment (start 51.5 40.0247) (end 51.5 38.5752) (width 0.25) (layer F.Cu) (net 5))
 (segment (start 45.6638 37.4979) (end 38.3412 30.1753) (width 0.25) (layer B.Cu) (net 5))
 (segment (start 38.3412 30.1753) (end 31.9832 30.1753) (width 0.25) (layer B.Cu) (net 5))
 (segment (start 31.9832 30.1753) (end 31.1753 29.3674) (width 0.25) (layer B.Cu) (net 5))
 (segment (start 31.1753 29.3674) (end 31.1753 29) (width 0.25) (layer B.Cu) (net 5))
 (segment (start 51.5 41.6) (end 51.5 40.0247) (width 0.25) (layer F.Cu) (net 5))
 (via (at 45.6638 37.4979) (size 0.8) (layers F.Cu B.Cu) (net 5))
 (segment (start 55.5 26.4) (end 55.5 27.9753) (width 0.25) (layer F.Cu) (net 10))
 (segment (start 55.5 27.9753) (end 60.4753 27.9753) (width 0.25) (layer F.Cu) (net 10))
 (segment (start 60.4753 27.9753) (end 61.5 29) (width 0.25) (layer F.Cu) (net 10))
 (segment (start 49.5 26.4) (end 49.5 27.9753) (width 0.25) (layer F.Cu) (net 9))
 (segment (start 49.5 27.9753) (end 51.6157 30.091) (width 0.25) (layer F.Cu) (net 9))
 (segment (start 51.6157 30.091) (end 63.1828 30.091) (width 0.25) (layer F.Cu) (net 9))
 (segment (start 63.1828 30.091) (end 63.9075 30.8157) (width 0.25) (layer F.Cu) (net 9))
 (segment (start 63.9075 30.8157) (end 63.9075 31) (width 0.25) (layer F.Cu) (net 9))
 (segment (start 55.5 41.6) (end 55.5 40.0247) (width 0.25) (layer F.Cu) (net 11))
 (segment (start 60.0247 41) (end 59.8799 40.8552) (width 0.25) (layer F.Cu) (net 11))
 (segment (start 59.8799 40.8552) (end 58.6305 40.8552) (width 0.25) (layer F.Cu) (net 11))
 (segment (start 56.1517 39.7496) (end 57.2573 40.8552) (width 0.25) (layer B.Cu) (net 11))
 (segment (start 57.2573 40.8552) (end 58.6305 40.8552) (width 0.25) (layer B.Cu) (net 11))
 (segment (start 61.1 41) (end 60.0247 41) (width 0.25) (layer F.Cu) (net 11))
 (segment (start 55.5 40.0247) (end 55.8766 40.0247) (width 0.25) (layer F.Cu) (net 11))
 (segment (start 55.8766 40.0247) (end 56.1517 39.7496) (width 0.25) (layer F.Cu) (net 11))
 (via (at 58.6305 40.8552) (size 0.8) (layers F.Cu B.Cu) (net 11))
 (via (at 56.1517 39.7496) (size 0.8) (layers F.Cu B.Cu) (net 11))
 (segment (start 43.5 41.6) (end 43.5 40.0247) (width 0.25) (layer F.Cu) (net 12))
 (segment (start 49.5 41.6) (end 49.5 39.8681) (width 0.25) (layer F.Cu) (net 12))
 (segment (start 49.5 39.8681) (end 48.8328 39.2009) (width 0.25) (layer F.Cu) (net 12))
 (segment (start 48.8328 39.2009) (end 44.3238 39.2009) (width 0.25) (layer F.Cu) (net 12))
 (segment (start 44.3238 39.2009) (end 43.5 40.0247) (width 0.25) (layer F.Cu) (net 12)))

